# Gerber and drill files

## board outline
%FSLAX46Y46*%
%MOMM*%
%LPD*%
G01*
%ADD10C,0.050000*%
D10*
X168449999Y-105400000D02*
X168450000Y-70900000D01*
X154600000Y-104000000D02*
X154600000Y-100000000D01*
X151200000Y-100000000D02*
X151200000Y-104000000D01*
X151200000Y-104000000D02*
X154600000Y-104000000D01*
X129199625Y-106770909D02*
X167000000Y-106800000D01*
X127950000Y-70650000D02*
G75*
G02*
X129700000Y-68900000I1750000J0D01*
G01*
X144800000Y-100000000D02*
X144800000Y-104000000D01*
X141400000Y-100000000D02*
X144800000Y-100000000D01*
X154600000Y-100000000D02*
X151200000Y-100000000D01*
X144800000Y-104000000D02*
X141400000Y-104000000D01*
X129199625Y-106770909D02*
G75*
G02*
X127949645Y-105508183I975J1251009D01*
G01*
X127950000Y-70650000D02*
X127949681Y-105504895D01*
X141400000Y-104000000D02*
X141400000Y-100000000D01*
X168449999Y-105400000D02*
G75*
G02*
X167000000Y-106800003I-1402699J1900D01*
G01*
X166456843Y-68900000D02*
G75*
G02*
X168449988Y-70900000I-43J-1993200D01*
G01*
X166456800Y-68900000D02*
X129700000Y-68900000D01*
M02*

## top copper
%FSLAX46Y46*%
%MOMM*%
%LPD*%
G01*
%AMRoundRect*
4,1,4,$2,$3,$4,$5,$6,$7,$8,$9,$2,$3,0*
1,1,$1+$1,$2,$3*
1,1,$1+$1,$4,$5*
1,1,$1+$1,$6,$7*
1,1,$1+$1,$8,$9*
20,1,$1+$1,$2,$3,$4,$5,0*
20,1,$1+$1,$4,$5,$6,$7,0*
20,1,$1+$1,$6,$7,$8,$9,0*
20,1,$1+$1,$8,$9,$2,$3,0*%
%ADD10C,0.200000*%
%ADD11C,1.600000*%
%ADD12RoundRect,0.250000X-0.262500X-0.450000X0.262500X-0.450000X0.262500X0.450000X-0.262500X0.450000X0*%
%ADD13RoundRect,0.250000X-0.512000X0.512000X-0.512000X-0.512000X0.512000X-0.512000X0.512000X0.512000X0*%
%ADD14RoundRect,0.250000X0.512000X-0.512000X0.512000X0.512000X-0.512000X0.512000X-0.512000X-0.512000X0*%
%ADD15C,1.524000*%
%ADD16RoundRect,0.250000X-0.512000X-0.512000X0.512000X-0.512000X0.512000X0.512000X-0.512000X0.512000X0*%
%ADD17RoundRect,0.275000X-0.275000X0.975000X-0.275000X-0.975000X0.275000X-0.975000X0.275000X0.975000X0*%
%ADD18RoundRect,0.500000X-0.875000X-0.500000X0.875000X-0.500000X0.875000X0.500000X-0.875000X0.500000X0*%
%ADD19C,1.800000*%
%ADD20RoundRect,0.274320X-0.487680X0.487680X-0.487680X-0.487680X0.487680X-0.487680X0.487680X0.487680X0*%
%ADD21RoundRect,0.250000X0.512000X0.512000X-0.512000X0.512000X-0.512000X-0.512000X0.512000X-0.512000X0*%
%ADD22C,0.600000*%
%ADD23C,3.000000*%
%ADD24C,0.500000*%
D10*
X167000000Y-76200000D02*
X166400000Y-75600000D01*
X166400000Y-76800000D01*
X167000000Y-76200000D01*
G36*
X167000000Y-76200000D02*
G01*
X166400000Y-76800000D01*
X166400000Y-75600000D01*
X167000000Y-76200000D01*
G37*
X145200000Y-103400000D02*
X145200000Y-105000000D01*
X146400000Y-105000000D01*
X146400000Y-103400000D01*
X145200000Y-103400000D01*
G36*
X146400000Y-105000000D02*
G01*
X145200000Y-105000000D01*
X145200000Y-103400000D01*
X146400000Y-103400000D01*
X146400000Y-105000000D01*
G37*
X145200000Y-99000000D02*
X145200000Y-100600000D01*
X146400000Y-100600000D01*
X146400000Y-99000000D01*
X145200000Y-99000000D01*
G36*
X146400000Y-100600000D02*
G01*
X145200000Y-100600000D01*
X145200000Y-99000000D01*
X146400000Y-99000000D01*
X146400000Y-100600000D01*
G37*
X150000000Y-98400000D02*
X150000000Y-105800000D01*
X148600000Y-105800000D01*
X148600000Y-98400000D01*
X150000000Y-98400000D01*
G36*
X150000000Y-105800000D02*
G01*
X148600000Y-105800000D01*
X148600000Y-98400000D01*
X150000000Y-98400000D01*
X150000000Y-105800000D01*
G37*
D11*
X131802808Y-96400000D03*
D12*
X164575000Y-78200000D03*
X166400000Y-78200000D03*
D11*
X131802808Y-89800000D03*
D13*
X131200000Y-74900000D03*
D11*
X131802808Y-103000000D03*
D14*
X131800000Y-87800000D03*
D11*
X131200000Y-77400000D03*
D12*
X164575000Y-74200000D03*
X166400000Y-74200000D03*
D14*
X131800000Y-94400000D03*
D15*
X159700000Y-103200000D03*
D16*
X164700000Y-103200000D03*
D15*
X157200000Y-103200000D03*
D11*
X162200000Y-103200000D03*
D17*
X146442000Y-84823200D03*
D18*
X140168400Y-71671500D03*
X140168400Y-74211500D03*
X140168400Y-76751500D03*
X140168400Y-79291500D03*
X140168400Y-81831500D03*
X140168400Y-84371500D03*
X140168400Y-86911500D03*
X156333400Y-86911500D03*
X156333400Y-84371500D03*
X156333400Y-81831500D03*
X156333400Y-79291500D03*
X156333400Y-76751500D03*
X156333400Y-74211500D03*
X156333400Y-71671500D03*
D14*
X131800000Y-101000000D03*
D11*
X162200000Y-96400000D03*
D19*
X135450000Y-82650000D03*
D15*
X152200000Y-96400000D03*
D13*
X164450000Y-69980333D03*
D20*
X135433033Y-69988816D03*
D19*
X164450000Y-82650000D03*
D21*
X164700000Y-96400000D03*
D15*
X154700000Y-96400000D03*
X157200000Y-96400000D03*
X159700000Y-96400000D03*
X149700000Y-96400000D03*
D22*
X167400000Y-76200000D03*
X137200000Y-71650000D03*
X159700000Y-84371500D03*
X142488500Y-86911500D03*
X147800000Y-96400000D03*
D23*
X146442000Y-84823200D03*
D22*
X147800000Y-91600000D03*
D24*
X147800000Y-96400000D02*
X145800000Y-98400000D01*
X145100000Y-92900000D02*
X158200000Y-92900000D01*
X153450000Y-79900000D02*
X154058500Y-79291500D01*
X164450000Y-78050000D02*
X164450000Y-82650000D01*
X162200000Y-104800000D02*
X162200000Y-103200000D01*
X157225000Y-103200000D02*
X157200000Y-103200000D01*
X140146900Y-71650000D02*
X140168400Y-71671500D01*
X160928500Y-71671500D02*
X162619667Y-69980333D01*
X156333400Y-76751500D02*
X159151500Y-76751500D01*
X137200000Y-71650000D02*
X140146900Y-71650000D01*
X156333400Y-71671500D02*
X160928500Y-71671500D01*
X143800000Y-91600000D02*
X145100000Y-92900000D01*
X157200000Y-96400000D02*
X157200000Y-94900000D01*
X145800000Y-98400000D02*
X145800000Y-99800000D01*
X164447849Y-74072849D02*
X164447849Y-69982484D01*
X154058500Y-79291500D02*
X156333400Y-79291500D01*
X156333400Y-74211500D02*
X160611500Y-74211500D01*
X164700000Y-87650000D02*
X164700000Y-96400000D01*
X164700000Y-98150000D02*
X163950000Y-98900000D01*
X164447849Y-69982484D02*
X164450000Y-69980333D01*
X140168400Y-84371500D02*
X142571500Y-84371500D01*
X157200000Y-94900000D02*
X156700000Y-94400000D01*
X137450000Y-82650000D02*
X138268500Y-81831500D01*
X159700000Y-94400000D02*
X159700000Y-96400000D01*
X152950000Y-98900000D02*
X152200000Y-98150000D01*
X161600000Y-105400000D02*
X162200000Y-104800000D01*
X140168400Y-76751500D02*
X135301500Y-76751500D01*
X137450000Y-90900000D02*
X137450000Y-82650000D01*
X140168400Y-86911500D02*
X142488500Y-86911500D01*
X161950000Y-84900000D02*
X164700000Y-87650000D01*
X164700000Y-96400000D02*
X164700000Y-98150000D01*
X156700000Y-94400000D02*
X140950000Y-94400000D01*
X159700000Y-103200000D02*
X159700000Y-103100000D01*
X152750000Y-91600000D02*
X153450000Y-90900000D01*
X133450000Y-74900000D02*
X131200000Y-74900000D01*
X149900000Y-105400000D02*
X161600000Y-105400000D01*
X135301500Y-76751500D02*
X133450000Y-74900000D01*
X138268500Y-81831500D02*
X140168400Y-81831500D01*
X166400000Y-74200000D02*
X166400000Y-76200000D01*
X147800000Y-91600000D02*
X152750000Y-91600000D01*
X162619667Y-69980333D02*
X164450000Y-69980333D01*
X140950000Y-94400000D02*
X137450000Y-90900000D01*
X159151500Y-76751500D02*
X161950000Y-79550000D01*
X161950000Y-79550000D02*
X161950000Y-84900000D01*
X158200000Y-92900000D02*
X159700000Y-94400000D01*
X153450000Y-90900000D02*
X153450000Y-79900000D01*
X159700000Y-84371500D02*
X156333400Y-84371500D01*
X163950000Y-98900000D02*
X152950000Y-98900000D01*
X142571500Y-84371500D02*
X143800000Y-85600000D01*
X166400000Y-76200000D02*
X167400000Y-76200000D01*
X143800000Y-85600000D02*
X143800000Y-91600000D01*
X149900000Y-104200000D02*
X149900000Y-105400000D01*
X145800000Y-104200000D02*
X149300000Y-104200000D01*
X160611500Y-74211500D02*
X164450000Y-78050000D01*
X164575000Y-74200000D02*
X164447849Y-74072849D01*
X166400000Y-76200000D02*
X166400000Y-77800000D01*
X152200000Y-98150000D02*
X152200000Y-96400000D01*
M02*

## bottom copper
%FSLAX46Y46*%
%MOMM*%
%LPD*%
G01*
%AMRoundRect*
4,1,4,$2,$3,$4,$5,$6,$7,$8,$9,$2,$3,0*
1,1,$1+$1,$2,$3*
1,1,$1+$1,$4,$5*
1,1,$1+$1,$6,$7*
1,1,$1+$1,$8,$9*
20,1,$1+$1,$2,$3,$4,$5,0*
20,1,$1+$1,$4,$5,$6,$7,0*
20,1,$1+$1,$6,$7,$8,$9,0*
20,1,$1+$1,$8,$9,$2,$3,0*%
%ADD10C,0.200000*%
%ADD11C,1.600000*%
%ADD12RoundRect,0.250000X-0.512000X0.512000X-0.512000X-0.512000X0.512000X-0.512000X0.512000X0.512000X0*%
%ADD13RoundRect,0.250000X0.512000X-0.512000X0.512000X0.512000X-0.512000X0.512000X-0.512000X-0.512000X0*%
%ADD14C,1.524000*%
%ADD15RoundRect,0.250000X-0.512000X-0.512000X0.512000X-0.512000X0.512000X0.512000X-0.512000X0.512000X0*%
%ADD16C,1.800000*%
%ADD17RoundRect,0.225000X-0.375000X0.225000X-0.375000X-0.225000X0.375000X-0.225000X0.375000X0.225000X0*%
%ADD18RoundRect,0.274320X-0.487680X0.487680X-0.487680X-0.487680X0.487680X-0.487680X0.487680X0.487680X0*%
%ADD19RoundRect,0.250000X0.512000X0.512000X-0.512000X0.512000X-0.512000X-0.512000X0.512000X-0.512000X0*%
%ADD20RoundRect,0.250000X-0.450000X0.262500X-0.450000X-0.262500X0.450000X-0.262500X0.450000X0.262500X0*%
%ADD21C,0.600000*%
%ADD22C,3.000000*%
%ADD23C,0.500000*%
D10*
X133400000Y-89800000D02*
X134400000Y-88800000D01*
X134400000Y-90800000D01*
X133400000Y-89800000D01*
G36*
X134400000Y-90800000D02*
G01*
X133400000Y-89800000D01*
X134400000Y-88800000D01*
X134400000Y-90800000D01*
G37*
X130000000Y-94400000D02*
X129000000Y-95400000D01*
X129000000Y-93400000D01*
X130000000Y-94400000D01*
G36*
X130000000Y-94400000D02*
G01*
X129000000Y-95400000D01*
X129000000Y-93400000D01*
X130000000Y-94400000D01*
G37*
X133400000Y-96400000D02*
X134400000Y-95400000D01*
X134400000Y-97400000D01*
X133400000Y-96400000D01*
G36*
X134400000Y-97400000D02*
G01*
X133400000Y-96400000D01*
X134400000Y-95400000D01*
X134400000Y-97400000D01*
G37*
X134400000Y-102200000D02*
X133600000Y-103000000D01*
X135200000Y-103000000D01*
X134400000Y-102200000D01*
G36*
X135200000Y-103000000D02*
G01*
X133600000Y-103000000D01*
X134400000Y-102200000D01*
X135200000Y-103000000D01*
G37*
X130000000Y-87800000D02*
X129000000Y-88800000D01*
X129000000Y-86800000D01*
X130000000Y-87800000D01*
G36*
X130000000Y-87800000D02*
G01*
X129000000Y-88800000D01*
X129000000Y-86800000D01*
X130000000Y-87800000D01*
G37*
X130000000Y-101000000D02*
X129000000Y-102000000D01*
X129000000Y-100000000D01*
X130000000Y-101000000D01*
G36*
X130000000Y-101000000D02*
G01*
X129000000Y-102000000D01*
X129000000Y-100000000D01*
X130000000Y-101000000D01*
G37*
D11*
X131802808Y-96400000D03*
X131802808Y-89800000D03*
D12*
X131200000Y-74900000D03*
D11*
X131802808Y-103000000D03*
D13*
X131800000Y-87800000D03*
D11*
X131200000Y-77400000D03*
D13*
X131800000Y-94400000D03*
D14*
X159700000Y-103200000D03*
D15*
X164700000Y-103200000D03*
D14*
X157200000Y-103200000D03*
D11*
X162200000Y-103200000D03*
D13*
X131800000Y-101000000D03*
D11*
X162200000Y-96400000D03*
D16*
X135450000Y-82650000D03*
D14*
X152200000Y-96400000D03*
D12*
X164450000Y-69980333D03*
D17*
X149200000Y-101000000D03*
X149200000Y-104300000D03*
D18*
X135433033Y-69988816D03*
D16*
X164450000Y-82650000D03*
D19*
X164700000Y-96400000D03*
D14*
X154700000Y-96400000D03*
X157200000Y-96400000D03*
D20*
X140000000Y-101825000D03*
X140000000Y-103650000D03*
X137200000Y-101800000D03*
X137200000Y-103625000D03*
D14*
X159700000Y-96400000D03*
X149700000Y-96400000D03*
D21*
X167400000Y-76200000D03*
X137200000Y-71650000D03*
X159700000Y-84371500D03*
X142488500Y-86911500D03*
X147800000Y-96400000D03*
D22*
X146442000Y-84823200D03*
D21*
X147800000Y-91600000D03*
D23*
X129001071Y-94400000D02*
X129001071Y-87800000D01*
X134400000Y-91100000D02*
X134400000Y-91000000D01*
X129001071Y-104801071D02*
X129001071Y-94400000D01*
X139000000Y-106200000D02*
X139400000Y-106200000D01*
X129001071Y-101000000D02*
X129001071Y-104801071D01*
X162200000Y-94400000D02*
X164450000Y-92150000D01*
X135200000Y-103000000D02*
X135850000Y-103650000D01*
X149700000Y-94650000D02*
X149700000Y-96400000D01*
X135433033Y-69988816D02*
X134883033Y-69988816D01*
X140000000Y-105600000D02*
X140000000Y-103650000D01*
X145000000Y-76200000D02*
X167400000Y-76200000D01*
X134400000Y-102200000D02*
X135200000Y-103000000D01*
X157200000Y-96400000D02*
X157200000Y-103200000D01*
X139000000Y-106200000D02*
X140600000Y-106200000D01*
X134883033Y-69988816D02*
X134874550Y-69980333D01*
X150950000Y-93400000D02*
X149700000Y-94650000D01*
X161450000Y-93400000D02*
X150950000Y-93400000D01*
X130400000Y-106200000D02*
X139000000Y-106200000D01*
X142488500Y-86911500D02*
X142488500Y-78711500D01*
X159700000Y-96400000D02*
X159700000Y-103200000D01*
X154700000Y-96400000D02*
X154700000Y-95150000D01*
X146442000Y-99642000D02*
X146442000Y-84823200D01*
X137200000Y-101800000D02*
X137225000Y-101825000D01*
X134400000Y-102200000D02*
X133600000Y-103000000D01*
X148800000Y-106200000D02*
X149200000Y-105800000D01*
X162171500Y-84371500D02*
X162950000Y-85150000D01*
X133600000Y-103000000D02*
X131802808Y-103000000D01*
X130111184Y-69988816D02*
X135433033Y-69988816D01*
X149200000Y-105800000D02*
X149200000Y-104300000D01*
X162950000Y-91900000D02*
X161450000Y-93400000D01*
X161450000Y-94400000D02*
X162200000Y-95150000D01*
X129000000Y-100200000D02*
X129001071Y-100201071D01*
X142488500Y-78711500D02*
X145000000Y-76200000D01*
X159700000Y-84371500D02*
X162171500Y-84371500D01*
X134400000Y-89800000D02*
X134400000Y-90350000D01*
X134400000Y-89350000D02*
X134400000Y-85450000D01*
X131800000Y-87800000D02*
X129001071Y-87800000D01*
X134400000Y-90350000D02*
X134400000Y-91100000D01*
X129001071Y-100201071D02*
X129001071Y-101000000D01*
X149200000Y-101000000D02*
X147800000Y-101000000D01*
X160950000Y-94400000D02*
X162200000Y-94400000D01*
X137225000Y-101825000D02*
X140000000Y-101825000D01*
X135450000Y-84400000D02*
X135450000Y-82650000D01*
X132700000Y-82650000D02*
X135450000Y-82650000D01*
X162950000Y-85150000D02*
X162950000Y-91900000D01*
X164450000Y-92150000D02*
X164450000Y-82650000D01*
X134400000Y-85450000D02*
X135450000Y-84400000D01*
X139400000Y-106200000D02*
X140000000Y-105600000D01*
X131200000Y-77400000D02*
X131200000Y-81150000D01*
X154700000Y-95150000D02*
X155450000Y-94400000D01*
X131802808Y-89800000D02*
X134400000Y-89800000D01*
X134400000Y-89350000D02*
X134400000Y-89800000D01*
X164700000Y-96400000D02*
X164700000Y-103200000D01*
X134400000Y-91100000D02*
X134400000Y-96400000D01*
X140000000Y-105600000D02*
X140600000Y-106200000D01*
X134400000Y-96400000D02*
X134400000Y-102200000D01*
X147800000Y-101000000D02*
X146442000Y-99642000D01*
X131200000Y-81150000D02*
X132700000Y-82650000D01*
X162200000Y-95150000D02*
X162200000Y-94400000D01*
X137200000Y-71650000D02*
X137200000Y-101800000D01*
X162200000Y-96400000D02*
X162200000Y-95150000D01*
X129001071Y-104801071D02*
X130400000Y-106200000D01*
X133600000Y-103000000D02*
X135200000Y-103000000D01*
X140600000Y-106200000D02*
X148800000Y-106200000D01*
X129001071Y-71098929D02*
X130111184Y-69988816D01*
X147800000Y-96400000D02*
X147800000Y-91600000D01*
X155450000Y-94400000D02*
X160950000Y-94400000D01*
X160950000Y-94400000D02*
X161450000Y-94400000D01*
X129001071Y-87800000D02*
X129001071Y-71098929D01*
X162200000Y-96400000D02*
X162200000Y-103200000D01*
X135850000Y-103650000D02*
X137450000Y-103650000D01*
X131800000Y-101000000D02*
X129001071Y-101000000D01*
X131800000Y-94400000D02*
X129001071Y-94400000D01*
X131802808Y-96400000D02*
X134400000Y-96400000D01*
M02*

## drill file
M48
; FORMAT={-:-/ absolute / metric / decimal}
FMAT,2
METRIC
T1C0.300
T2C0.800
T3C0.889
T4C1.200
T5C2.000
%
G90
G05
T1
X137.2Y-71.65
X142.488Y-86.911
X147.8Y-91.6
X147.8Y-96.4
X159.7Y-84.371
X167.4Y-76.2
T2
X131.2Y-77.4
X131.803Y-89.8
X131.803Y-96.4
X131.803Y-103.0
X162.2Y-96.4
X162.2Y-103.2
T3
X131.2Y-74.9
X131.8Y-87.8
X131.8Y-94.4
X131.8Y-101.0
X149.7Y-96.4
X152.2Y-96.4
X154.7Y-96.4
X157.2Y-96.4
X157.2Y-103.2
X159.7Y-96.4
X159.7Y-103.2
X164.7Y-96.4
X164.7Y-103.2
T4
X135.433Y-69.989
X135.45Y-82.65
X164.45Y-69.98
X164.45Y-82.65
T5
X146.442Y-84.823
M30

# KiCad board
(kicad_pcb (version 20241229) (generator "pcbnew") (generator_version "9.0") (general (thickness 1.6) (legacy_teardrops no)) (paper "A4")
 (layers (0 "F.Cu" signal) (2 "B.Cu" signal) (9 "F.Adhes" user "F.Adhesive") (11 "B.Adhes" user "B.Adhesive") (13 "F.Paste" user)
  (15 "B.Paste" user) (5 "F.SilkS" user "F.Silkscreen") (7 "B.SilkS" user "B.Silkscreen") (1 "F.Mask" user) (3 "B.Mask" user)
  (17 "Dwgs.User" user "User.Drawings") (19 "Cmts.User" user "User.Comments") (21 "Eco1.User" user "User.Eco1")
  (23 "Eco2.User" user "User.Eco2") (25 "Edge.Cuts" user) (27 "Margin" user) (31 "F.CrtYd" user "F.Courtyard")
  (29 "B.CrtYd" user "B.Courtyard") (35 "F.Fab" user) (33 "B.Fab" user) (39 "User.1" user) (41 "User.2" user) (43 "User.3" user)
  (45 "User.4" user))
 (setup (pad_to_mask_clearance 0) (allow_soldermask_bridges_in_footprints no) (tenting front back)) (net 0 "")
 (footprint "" (layer "F.Cu") (at 131.802808 96.4 180)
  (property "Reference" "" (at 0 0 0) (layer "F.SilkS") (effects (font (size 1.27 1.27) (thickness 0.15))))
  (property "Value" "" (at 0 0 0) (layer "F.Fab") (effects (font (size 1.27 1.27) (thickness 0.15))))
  (pad "GND" thru_hole circle (at 0 0 90) (size 1.6 1.6) (drill 0.8) (layers "*.Cu" "*.Mask") (remove_unused_layers no)))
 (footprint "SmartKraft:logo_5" (layer "F.Cu") (at 163.6 87)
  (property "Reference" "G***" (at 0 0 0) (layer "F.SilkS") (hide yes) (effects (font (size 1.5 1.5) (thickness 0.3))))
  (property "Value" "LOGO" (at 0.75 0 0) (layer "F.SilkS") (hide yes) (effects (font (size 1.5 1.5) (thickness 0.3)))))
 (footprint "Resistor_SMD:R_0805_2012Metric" (layer "F.Cu") (at 165.4875 78.2)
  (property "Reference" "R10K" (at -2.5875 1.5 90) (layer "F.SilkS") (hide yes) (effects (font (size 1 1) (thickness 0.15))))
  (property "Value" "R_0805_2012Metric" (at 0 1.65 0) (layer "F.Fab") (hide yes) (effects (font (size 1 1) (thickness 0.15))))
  (pad "1" smd roundrect (at -0.9125 0) (size 1.025 1.4) (layers "F.Cu" "F.Mask" "F.Paste") (roundrect_rratio 0.243902))
  (pad "2" smd roundrect (at 0.9125 0) (size 1.025 1.4) (layers "F.Cu" "F.Mask" "F.Paste") (roundrect_rratio 0.243902)))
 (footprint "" (layer "F.Cu") (at 131.802808 89.8 180)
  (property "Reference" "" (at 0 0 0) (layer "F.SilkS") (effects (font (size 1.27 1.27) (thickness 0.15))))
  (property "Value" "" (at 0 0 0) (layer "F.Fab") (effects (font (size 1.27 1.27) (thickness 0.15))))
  (pad "GND" thru_hole circle (at 0 0 90) (size 1.6 1.6) (drill 0.8) (layers "*.Cu" "*.Mask") (remove_unused_layers no)))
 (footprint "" (layer "F.Cu") (at 131.2 74.9 -90)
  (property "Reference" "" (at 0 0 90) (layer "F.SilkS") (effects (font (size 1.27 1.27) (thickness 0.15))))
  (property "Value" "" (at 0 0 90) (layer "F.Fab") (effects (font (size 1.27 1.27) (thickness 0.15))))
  (pad "+" thru_hole roundrect (at 0 0 270) (size 1.524 1.524) (drill 0.889) (layers "*.Cu" "*.Mask") (remove_unused_layers no)
   (roundrect_rratio 0.1640419948)))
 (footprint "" (layer "F.Cu") (at 131.802808 103 180)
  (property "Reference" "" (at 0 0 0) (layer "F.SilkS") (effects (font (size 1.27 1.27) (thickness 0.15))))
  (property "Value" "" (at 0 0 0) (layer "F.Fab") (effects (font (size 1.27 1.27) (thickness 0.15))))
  (pad "GND" thru_hole circle (at 0 0 90) (size 1.6 1.6) (drill 0.8) (layers "*.Cu" "*.Mask") (remove_unused_layers no)))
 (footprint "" (layer "F.Cu") (at 131.8 87.8 180)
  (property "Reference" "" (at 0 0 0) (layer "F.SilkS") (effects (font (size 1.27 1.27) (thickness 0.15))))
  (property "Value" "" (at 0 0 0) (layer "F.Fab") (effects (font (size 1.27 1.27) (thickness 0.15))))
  (pad "+" thru_hole roundrect (at 0 0 90) (size 1.524 1.524) (drill 0.889) (layers "*.Cu" "*.Mask") (remove_unused_layers no)
   (roundrect_rratio 0.1640419948)))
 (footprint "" (layer "F.Cu") (at 131.2 77.4 -90)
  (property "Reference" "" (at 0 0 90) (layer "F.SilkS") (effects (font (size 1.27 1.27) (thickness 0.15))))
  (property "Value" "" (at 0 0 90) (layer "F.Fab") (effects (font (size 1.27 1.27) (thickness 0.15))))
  (pad "GND" thru_hole circle (at 0 0 270) (size 1.6 1.6) (drill 0.8) (layers "*.Cu" "*.Mask") (remove_unused_layers no)))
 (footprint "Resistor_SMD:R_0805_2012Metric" (layer "F.Cu") (at 165.4875 74.2)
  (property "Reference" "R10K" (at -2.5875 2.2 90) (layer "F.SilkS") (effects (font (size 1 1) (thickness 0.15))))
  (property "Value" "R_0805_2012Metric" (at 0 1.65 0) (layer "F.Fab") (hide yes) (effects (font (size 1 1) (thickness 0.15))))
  (pad "1" smd roundrect (at -0.9125 0) (size 1.025 1.4) (layers "F.Cu" "F.Mask" "F.Paste") (roundrect_rratio 0.243902))
  (pad "2" smd roundrect (at 0.9125 0) (size 1.025 1.4) (layers "F.Cu" "F.Mask" "F.Paste") (roundrect_rratio 0.243902)))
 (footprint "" (layer "F.Cu") (at 131.8 94.4 180)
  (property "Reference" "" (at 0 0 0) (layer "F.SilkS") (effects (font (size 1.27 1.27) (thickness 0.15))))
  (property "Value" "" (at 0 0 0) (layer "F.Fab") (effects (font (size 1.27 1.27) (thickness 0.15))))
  (pad "+" thru_hole roundrect (at 0 0 90) (size 1.524 1.524) (drill 0.889) (layers "*.Cu" "*.Mask") (remove_unused_layers no)
   (roundrect_rratio 0.1640419948)))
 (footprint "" (layer "F.Cu") (at 159.7 103.2)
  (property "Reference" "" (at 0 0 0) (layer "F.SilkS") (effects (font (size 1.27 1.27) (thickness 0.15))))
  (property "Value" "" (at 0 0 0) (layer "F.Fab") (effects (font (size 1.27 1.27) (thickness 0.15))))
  (pad "SCL" thru_hole circle (at 0 0) (size 1.524 1.524) (drill 0.889) (layers "*.Cu" "*.Mask") (remove_unused_layers no)))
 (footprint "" (layer "F.Cu") (at 164.7 103.2)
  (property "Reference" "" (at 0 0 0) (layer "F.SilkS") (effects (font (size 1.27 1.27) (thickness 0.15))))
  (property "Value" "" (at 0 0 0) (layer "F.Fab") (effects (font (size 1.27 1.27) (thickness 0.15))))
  (pad "3.3V" thru_hole roundrect (at 0 0) (size 1.524 1.524) (drill 0.889) (layers "*.Cu" "*.Mask") (remove_unused_layers no)
   (roundrect_rratio 0.1640419948)))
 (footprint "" (layer "F.Cu") (at 157.2 103.2)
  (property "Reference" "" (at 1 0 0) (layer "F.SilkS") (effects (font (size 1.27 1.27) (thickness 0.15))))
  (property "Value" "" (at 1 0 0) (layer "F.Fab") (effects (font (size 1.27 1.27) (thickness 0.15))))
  (pad "SDA" thru_hole circle (at 0 0) (size 1.524 1.524) (drill 0.889) (layers "*.Cu" "*.Mask") (remove_unused_layers no)))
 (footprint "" (layer "F.Cu") (at 162.2 103.2)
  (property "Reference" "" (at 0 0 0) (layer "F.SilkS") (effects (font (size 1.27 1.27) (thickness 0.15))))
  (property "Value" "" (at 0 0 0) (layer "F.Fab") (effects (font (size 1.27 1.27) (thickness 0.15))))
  (pad "GND" thru_hole circle (at 0 0) (size 1.6 1.6) (drill 0.8) (layers "*.Cu" "*.Mask") (remove_unused_layers no)))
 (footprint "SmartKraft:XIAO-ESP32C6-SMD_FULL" (layer "F.Cu") (at 148.45 79.27)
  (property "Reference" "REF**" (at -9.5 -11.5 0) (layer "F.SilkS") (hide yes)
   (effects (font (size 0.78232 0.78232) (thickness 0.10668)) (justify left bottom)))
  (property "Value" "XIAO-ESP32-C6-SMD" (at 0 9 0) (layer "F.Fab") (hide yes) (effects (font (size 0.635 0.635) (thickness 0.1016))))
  (pad "" smd circle (at -1.5 -8.62) (size 1.7 1.7) (layers)) (pad "" smd circle (at -1.5 -6.08) (size 1.7 1.7) (layers))
  (pad "" smd circle (at -1.5 -3.54) (size 1.7 1.7) (layers)) (pad "" smd circle (at -1.5 -1) (size 1.7 1.7) (layers))
  (pad "" smd roundrect (at 0.532 5.5532 270) (size 2.5 1.1) (layers) (roundrect_rratio 0.25) (solder_mask_margin 0.0508)
   (thermal_bridge_angle 45))
  (pad "" smd circle (at 0.9474 -1.0568) (size 1.7 1.7) (layers)) (pad "" smd circle (at 1.04 -8.62) (size 1.7 1.7) (layers))
  (pad "" smd circle (at 1.04 -6.08) (size 1.7 1.7) (layers)) (pad "" smd circle (at 1.04 -3.54) (size 1.7 1.7) (layers))
  (pad "+" smd roundrect (at -2.008 5.5532 270) (size 2.5 1.1) (layers "F.Cu" "F.Mask") (roundrect_rratio 0.25) (solder_mask_margin 0.0508)
   (thermal_bridge_angle 45))
  (pad "1" smd roundrect (at -8.2816 -7.5985) (size 2.75 2) (layers "F.Cu" "F.Mask") (roundrect_rratio 0.25) (solder_mask_margin 0.0508)
   (thermal_bridge_angle 45))
  (pad "2" smd roundrect (at -8.2816 -5.0585) (size 2.75 2) (layers "F.Cu" "F.Mask") (roundrect_rratio 0.25) (solder_mask_margin 0.0508)
   (thermal_bridge_angle 45))
  (pad "3" smd roundrect (at -8.2816 -2.5185) (size 2.75 2) (layers "F.Cu" "F.Mask") (roundrect_rratio 0.25) (solder_mask_margin 0.0508)
   (thermal_bridge_angle 45))
  (pad "4" smd roundrect (at -8.2816 0.0215) (size 2.75 2) (layers "F.Cu" "F.Mask") (roundrect_rratio 0.25) (solder_mask_margin 0.0508)
   (thermal_bridge_angle 45))
  (pad "5" smd roundrect (at -8.2816 2.5615) (size 2.75 2) (layers "F.Cu" "F.Mask") (roundrect_rratio 0.25) (solder_mask_margin 0.0508)
   (thermal_bridge_angle 45))
  (pad "6" smd roundrect (at -8.2816 5.1015) (size 2.75 2) (layers "F.Cu" "F.Mask") (roundrect_rratio 0.25) (solder_mask_margin 0.0508)
   (thermal_bridge_angle 45))
  (pad "7" smd roundrect (at -8.2816 7.6415) (size 2.75 2) (layers "F.Cu" "F.Mask") (roundrect_rratio 0.25) (solder_mask_margin 0.0508)
   (thermal_bridge_angle 45))
  (pad "8" smd roundrect (at 7.8834 7.6415) (size 2.75 2) (layers "F.Cu" "F.Mask") (roundrect_rratio 0.25) (solder_mask_margin 0.0508)
   (thermal_bridge_angle 45))
  (pad "9" smd roundrect (at 7.8834 5.1015) (size 2.75 2) (layers "F.Cu" "F.Mask") (roundrect_rratio 0.25) (solder_mask_margin 0.0508)
   (thermal_bridge_angle 45))
  (pad "10" smd roundrect (at 7.8834 2.5615) (size 2.75 2) (layers "F.Cu" "F.Mask") (roundrect_rratio 0.25) (solder_mask_margin 0.0508)
   (thermal_bridge_angle 45))
  (pad "11" smd roundrect (at 7.8834 0.0215) (size 2.75 2) (layers "F.Cu" "F.Mask") (roundrect_rratio 0.25) (solder_mask_margin 0.0508)
   (thermal_bridge_angle 45))
  (pad "12" smd roundrect (at 7.8834 -2.5185) (size 2.75 2) (layers "F.Cu" "F.Mask") (roundrect_rratio 0.25) (solder_mask_margin 0.0508)
   (thermal_bridge_angle 45))
  (pad "13" smd roundrect (at 7.8834 -5.0585) (size 2.75 2) (layers "F.Cu" "F.Mask") (roundrect_rratio 0.25) (solder_mask_margin 0.0508)
   (thermal_bridge_angle 45))
  (pad "14" smd roundrect (at 7.8834 -7.5985) (size 2.75 2) (layers "F.Cu" "F.Mask") (roundrect_rratio 0.25) (solder_mask_margin 0.0508)
   (thermal_bridge_angle 45)))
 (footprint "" (layer "F.Cu") (at 131.8 101 180)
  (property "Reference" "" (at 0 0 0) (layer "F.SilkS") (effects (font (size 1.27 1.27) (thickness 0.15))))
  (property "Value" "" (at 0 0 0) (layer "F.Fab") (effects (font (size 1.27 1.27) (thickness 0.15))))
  (pad "+" thru_hole roundrect (at 0 0 90) (size 1.524 1.524) (drill 0.889) (layers "*.Cu" "*.Mask") (remove_unused_layers no)
   (roundrect_rratio 0.1640419948)))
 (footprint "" (layer "B.Cu") (at 162.2 96.4)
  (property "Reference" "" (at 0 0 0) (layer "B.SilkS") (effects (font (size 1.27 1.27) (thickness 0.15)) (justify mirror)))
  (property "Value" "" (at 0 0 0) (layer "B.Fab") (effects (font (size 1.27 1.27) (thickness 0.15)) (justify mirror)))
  (pad "GND" thru_hole circle (at 0 0) (size 1.6 1.6) (drill 0.8) (layers "*.Cu" "*.Mask") (remove_unused_layers no)))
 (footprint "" (layer "B.Cu") (at 135.45 82.65 -90)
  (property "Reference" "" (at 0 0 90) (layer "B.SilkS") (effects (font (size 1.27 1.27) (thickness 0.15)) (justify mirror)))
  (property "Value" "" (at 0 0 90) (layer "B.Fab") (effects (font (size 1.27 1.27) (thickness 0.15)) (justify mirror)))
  (pad "GND" thru_hole circle (at 0 0 270) (size 1.8 1.8) (drill 1.2) (layers "*.Cu" "*.Mask") (remove_unused_layers no)))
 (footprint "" (layer "B.Cu") (at 152.2 96.4)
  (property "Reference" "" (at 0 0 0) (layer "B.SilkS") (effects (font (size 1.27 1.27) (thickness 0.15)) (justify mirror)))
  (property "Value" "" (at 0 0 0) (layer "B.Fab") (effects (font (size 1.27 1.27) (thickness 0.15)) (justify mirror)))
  (pad "CS" thru_hole circle (at 0 0) (size 1.524 1.524) (drill 0.889) (layers "*.Cu" "*.Mask") (remove_unused_layers no)))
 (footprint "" (layer "B.Cu") (at 164.45 69.980333 -90)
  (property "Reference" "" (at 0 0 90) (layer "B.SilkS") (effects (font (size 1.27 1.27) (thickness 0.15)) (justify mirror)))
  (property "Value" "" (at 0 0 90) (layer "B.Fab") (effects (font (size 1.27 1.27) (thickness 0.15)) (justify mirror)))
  (pad "+" thru_hole roundrect (at 0 0 270) (size 1.524 1.524) (drill 1.2) (layers "*.Cu" "*.Mask") (remove_unused_layers no)
   (roundrect_rratio 0.1640419948)))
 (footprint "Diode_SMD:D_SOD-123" (layer "B.Cu") (at 149.2 102.65 -90)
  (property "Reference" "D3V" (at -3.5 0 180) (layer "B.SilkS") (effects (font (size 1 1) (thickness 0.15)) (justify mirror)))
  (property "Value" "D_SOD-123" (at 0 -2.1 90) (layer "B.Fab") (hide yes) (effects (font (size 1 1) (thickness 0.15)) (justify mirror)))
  (pad "1" smd roundrect (at -1.65 0 270) (size 0.9 1.2) (layers "B.Cu" "B.Mask" "B.Paste") (roundrect_rratio 0.25))
  (pad "2" smd roundrect (at 1.65 0 270) (size 0.9 1.2) (layers "B.Cu" "B.Mask" "B.Paste") (roundrect_rratio 0.25)))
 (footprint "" (layer "B.Cu") (at 135.433033 69.988816 -90)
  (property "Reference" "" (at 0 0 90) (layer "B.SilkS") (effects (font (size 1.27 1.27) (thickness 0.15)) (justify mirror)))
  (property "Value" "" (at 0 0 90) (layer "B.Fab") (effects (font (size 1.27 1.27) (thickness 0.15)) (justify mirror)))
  (pad "+" thru_hole roundrect (at 0 0 270) (size 1.524 1.524) (drill 1.2) (layers "*.Cu" "*.Mask") (remove_unused_layers no)
   (roundrect_rratio 0.18)))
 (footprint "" (layer "B.Cu") (at 164.45 82.65 -90)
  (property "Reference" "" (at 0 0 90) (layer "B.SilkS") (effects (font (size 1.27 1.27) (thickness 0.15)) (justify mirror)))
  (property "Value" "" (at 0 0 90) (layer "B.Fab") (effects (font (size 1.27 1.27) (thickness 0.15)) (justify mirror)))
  (pad "GND" thru_hole circle (at 0 0 270) (size 1.8 1.8) (drill 1.2) (layers "*.Cu" "*.Mask") (remove_unused_layers no)))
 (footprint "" (layer "B.Cu") (at 164.7 96.4 -90)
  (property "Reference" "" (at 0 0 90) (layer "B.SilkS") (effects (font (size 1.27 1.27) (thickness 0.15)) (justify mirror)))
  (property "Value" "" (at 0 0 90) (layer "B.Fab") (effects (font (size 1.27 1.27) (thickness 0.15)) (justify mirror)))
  (pad "3.3V" thru_hole roundrect (at 0 0 180) (size 1.524 1.524) (drill 0.889) (layers "*.Cu" "*.Mask") (remove_unused_layers no)
   (roundrect_rratio 0.1640419948)))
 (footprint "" (layer "B.Cu") (at 154.7 96.4)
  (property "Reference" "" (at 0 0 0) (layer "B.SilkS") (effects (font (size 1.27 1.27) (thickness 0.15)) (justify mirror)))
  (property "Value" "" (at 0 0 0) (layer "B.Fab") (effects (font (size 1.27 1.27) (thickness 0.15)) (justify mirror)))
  (pad "SDO" thru_hole circle (at 0 0) (size 1.524 1.524) (drill 0.889) (layers "*.Cu" "*.Mask") (remove_unused_layers no)))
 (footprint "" (layer "B.Cu") (at 157.2 96.4)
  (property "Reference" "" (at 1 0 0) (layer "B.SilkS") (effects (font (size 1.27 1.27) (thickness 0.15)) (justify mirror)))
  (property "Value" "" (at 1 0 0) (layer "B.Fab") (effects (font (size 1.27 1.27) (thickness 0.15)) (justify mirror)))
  (pad "SDA" thru_hole circle (at 0 0) (size 1.524 1.524) (drill 0.889) (layers "*.Cu" "*.Mask") (remove_unused_layers no)))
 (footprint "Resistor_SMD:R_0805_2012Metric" (layer "B.Cu") (at 140 102.7375 -90)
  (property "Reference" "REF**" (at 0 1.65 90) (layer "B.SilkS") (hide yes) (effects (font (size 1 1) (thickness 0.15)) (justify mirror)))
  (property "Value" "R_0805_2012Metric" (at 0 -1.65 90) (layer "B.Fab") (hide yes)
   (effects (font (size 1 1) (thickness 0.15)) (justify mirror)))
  (pad "1" smd roundrect (at -0.9125 0 270) (size 1.025 1.4) (layers "B.Cu" "B.Mask" "B.Paste") (roundrect_rratio 0.243902))
  (pad "2" smd roundrect (at 0.9125 0 270) (size 1.025 1.4) (layers "B.Cu" "B.Mask" "B.Paste") (roundrect_rratio 0.243902)))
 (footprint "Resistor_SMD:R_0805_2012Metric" (layer "B.Cu") (at 137.2 102.7125 -90)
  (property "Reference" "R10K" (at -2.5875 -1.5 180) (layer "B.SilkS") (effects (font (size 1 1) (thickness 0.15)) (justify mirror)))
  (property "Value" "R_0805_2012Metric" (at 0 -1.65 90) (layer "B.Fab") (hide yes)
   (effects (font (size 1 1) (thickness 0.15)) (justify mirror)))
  (pad "1" smd roundrect (at -0.9125 0 270) (size 1.025 1.4) (layers "B.Cu" "B.Mask" "B.Paste") (roundrect_rratio 0.243902))
  (pad "2" smd roundrect (at 0.9125 0 270) (size 1.025 1.4) (layers "B.Cu" "B.Mask" "B.Paste") (roundrect_rratio 0.243902)))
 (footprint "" (layer "B.Cu") (at 159.7 96.4)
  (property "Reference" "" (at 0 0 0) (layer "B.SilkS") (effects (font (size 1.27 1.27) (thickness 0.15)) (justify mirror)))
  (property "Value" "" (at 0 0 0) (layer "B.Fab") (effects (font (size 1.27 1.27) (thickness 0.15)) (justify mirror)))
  (pad "SCL" thru_hole circle (at 0 0) (size 1.524 1.524) (drill 0.889) (layers "*.Cu" "*.Mask") (remove_unused_layers no)))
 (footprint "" (layer "B.Cu") (at 149.7 96.4)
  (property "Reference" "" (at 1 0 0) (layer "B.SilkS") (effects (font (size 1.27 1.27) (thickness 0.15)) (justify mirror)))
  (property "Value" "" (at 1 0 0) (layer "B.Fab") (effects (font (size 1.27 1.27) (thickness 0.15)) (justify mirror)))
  (pad "INT" thru_hole circle (at 0 0) (size 1.524 1.524) (drill 0.889) (layers "*.Cu" "*.Mask") (remove_unused_layers no)))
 (gr_poly (pts (xy 167 76.2) (xy 166.4 75.6) (xy 166.4 76.8)) (stroke (width 0.2) (type solid)) (fill yes) (layer "F.Cu"))
 (gr_poly
  (pts (xy 145.2 103.4) (xy 145.2 105) (xy 146.4 105) (xy 146.4 103.4)) (stroke (width 0.2) (type solid)) (fill yes)
  (layers "F.Cu" "F.Mask"))
 (gr_poly
  (pts (xy 145.2 99) (xy 145.2 100.6) (xy 146.4 100.6) (xy 146.4 99)) (stroke (width 0.2) (type solid)) (fill yes) (layers "F.Cu" "F.Mask"))
 (gr_poly
  (pts (xy 150 98.4) (xy 150 105.8) (xy 148.6 105.8) (xy 148.6 98.4)) (stroke (width 0.2) (type solid)) (fill yes) (layers "F.Cu" "F.Mask"))
 (gr_poly (pts (xy 133.4 89.8) (xy 134.4 88.8) (xy 134.4 90.8)) (stroke (width 0.2) (type solid)) (fill yes) (layer "B.Cu"))
 (gr_poly (pts (xy 130 94.4) (xy 129 95.4) (xy 129 93.4)) (stroke (width 0.2) (type solid)) (fill yes) (layer "B.Cu"))
 (gr_poly (pts (xy 133.4 96.4) (xy 134.4 95.4) (xy 134.4 97.4)) (stroke (width 0.2) (type solid)) (fill yes) (layer "B.Cu"))
 (gr_poly (pts (xy 134.4 102.2) (xy 133.6 103) (xy 135.2 103)) (stroke (width 0.2) (type solid)) (fill yes) (layer "B.Cu"))
 (gr_poly (pts (xy 130 87.8) (xy 129 88.8) (xy 129 86.8)) (stroke (width 0.2) (type solid)) (fill yes) (layer "B.Cu"))
 (gr_poly (pts (xy 130 101) (xy 129 102) (xy 129 100)) (stroke (width 0.2) (type solid)) (fill yes) (layer "B.Cu"))
 (gr_line (start 168.449999 105.4) (end 168.45 70.9) (stroke (width 0.05) (type default)) (layer "Edge.Cuts"))
 (gr_line (start 154.6 104) (end 154.6 100) (stroke (width 0.05) (type default)) (layer "Edge.Cuts"))
 (gr_line (start 151.2 100) (end 151.2 104) (stroke (width 0.05) (type default)) (layer "Edge.Cuts"))
 (gr_line (start 151.2 104) (end 154.6 104) (stroke (width 0.05) (type default)) (layer "Edge.Cuts"))
 (gr_line (start 129.199625 106.770909) (end 167 106.8) (stroke (width 0.05) (type default)) (layer "Edge.Cuts"))
 (gr_arc (start 127.95 70.65) (mid 128.462563 69.412563) (end 129.7 68.9) (stroke (width 0.05) (type default)) (layer "Edge.Cuts"))
 (gr_line (start 144.8 100) (end 144.8 104) (stroke (width 0.05) (type default)) (layer "Edge.Cuts"))
 (gr_line (start 141.4 100) (end 144.8 100) (stroke (width 0.05) (type default)) (layer "Edge.Cuts"))
 (gr_line (start 154.6 100) (end 151.2 100) (stroke (width 0.05) (type default)) (layer "Edge.Cuts"))
 (gr_line (start 144.8 104) (end 141.4 104) (stroke (width 0.05) (type default)) (layer "Edge.Cuts"))
 (gr_arc (start 129.199625 106.770909) (mid 128.311535 106.4) (end 127.949681 105.508183) (stroke (width 0.05) (type default))
  (layer "Edge.Cuts"))
 (gr_line (start 127.95 70.65) (end 127.949681 105.504895) (stroke (width 0.05) (type default)) (layer "Edge.Cuts"))
 (gr_line (start 141.4 104) (end 141.4 100) (stroke (width 0.05) (type default)) (layer "Edge.Cuts"))
 (gr_arc (start 168.449999 105.4) (mid 168.021618 106.407212) (end 167 106.8) (stroke (width 0.05) (type default)) (layer "Edge.Cuts"))
 (gr_arc (start 166.456843 68.9) (mid 167.868639 69.486203) (end 168.45 70.9) (stroke (width 0.05) (type default)) (layer "Edge.Cuts"))
 (gr_line (start 166.4568 68.9) (end 129.7 68.9) (stroke (width 0.05) (type default)) (layer "Edge.Cuts"))
 (segment (start 147.8 96.4) (end 145.8 98.4) (width 0.5) (layer "F.Cu") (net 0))
 (segment (start 145.1 92.9) (end 158.2 92.9) (width 0.5) (layer "F.Cu") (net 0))
 (segment (start 153.45 79.9) (end 154.0585 79.2915) (width 0.5) (layer "F.Cu") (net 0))
 (segment (start 164.45 78.05) (end 164.45 82.65) (width 0.5) (layer "F.Cu") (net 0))
 (segment (start 162.2 104.8) (end 162.2 103.2) (width 0.5) (layer "F.Cu") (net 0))
 (segment (start 157.225 103.2) (end 157.2 103.2) (width 0.5) (layer "F.Cu") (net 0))
 (segment (start 140.1469 71.65) (end 140.1684 71.6715) (width 0.5) (layer "F.Cu") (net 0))
 (segment (start 160.9285 71.6715) (end 162.619667 69.980333) (width 0.5) (layer "F.Cu") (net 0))
 (segment (start 156.3334 76.7515) (end 159.1515 76.7515) (width 0.5) (layer "F.Cu") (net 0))
 (segment (start 137.2 71.65) (end 140.1469 71.65) (width 0.5) (layer "F.Cu") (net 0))
 (segment (start 156.3334 71.6715) (end 160.9285 71.6715) (width 0.5) (layer "F.Cu") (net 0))
 (segment (start 143.8 91.6) (end 145.1 92.9) (width 0.5) (layer "F.Cu") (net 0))
 (segment (start 157.2 96.4) (end 157.2 94.9) (width 0.5) (layer "F.Cu") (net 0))
 (segment (start 145.8 98.4) (end 145.8 99.8) (width 0.5) (layer "F.Cu") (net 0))
 (segment (start 164.447849 74.072849) (end 164.447849 69.982484) (width 0.5) (layer "F.Cu") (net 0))
 (segment (start 154.0585 79.2915) (end 156.3334 79.2915) (width 0.5) (layer "F.Cu") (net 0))
 (segment (start 156.3334 74.2115) (end 160.6115 74.2115) (width 0.5) (layer "F.Cu") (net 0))
 (segment (start 164.7 87.65) (end 164.7 96.4) (width 0.5) (layer "F.Cu") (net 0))
 (segment (start 164.7 98.15) (end 163.95 98.9) (width 0.5) (layer "F.Cu") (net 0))
 (segment (start 164.447849 69.982484) (end 164.45 69.980333) (width 0.5) (layer "F.Cu") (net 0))
 (segment (start 140.1684 84.3715) (end 142.5715 84.3715) (width 0.5) (layer "F.Cu") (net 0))
 (segment (start 157.2 94.9) (end 156.7 94.4) (width 0.5) (layer "F.Cu") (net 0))
 (segment (start 137.45 82.65) (end 138.2685 81.8315) (width 0.5) (layer "F.Cu") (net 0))
 (segment (start 159.7 94.4) (end 159.7 96.4) (width 0.5) (layer "F.Cu") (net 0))
 (segment (start 152.95 98.9) (end 152.2 98.15) (width 0.5) (layer "F.Cu") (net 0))
 (segment (start 161.6 105.4) (end 162.2 104.8) (width 0.5) (layer "F.Cu") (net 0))
 (segment (start 140.1684 76.7515) (end 135.3015 76.7515) (width 0.5) (layer "F.Cu") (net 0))
 (segment (start 137.45 90.9) (end 137.45 82.65) (width 0.5) (layer "F.Cu") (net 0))
 (segment (start 140.1684 86.9115) (end 142.4885 86.9115) (width 0.5) (layer "F.Cu") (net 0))
 (segment (start 161.95 84.9) (end 164.7 87.65) (width 0.5) (layer "F.Cu") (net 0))
 (segment (start 164.7 96.4) (end 164.7 98.15) (width 0.5) (layer "F.Cu") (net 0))
 (segment (start 156.7 94.4) (end 140.95 94.4) (width 0.5) (layer "F.Cu") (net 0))
 (segment (start 159.7 103.2) (end 159.7 103.1) (width 0.5) (layer "F.Cu") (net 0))
 (segment (start 152.75 91.6) (end 153.45 90.9) (width 0.5) (layer "F.Cu") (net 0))
 (segment (start 133.45 74.9) (end 131.2 74.9) (width 0.5) (layer "F.Cu") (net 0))
 (segment (start 149.9 105.4) (end 161.6 105.4) (width 0.5) (layer "F.Cu") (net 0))
 (segment (start 135.3015 76.7515) (end 133.45 74.9) (width 0.5) (layer "F.Cu") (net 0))
 (segment (start 138.2685 81.8315) (end 140.1684 81.8315) (width 0.5) (layer "F.Cu") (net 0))
 (segment (start 166.4 74.2) (end 166.4 76.2) (width 0.5) (layer "F.Cu") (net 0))
 (segment (start 147.8 91.6) (end 152.75 91.6) (width 0.5) (layer "F.Cu") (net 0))
 (segment (start 162.619667 69.980333) (end 164.45 69.980333) (width 0.5) (layer "F.Cu") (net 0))
 (segment (start 140.95 94.4) (end 137.45 90.9) (width 0.5) (layer "F.Cu") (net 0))
 (segment (start 159.1515 76.7515) (end 161.95 79.55) (width 0.5) (layer "F.Cu") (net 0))
 (segment (start 161.95 79.55) (end 161.95 84.9) (width 0.5) (layer "F.Cu") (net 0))
 (segment (start 158.2 92.9) (end 159.7 94.4) (width 0.5) (layer "F.Cu") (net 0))
 (segment (start 153.45 90.9) (end 153.45 79.9) (width 0.5) (layer "F.Cu") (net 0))
 (segment (start 159.7 84.3715) (end 156.3334 84.3715) (width 0.5) (layer "F.Cu") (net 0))
 (segment (start 163.95 98.9) (end 152.95 98.9) (width 0.5) (layer "F.Cu") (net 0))
 (segment (start 142.5715 84.3715) (end 143.8 85.6) (width 0.5) (layer "F.Cu") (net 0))
 (segment (start 166.4 76.2) (end 167.4 76.2) (width 0.5) (layer "F.Cu") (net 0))
 (segment (start 143.8 85.6) (end 143.8 91.6) (width 0.5) (layer "F.Cu") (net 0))
 (segment (start 149.9 104.2) (end 149.9 105.4) (width 0.5) (layer "F.Cu") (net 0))
 (segment (start 145.8 104.2) (end 149.3 104.2) (width 0.5) (layer "F.Cu") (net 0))
 (segment (start 160.6115 74.2115) (end 164.45 78.05) (width 0.5) (layer "F.Cu") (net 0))
 (segment (start 164.575 74.2) (end 164.447849 74.072849) (width 0.5) (layer "F.Cu") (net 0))
 (segment (start 166.4 76.2) (end 166.4 77.8) (width 0.5) (layer "F.Cu") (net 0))
 (segment (start 152.2 98.15) (end 152.2 96.4) (width 0.5) (layer "F.Cu") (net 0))
 (via (at 167.4 76.2) (size 0.6) (drill 0.3) (layers "F.Cu" "B.Cu") (tenting none) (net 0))
 (via (at 137.2 71.65) (size 0.6) (drill 0.3) (layers "F.Cu" "B.Cu") (tenting none) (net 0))
 (via (at 159.7 84.3715) (size 0.6) (drill 0.3) (layers "F.Cu" "B.Cu") (tenting none) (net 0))
 (via (at 142.4885 86.9115) (size 0.6) (drill 0.3) (layers "F.Cu" "B.Cu") (tenting none) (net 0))
 (via (at 147.8 96.4) (size 0.6) (drill 0.3) (layers "F.Cu" "B.Cu") (tenting none) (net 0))
 (via (at 146.442 84.8232) (size 3) (drill 2) (layers "F.Cu" "B.Cu") (tenting none) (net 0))
 (via (at 147.8 91.6) (size 0.6) (drill 0.3) (layers "F.Cu" "B.Cu") (tenting none) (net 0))
 (segment (start 129.001071 94.4) (end 129.001071 87.8) (width 0.5) (layer "B.Cu") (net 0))
 (segment (start 134.4 91.1) (end 134.4 91) (width 0.5) (layer "B.Cu") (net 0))
 (segment (start 129.001071 104.801071) (end 129.001071 94.4) (width 0.5) (layer "B.Cu") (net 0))
 (segment (start 139 106.2) (end 139.4 106.2) (width 0.5) (layer "B.Cu") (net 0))
 (segment (start 129.001071 101) (end 129.001071 104.801071) (width 0.5) (layer "B.Cu") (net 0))
 (segment (start 162.2 94.4) (end 164.45 92.15) (width 0.5) (layer "B.Cu") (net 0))
 (segment (start 135.2 103) (end 135.85 103.65) (width 0.5) (layer "B.Cu") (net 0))
 (segment (start 149.7 94.65) (end 149.7 96.4) (width 0.5) (layer "B.Cu") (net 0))
 (segment (start 135.433033 69.988816) (end 134.883033 69.988816) (width 0.5) (layer "B.Cu") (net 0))
 (segment (start 140 105.6) (end 140 103.65) (width 0.5) (layer "B.Cu") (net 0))
 (segment (start 145 76.2) (end 167.4 76.2) (width 0.5) (layer "B.Cu") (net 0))
 (segment (start 134.4 102.2) (end 135.2 103) (width 0.5) (layer "B.Cu") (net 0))
 (segment (start 157.2 96.4) (end 157.2 103.2) (width 0.5) (layer "B.Cu") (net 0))
 (segment (start 139 106.2) (end 140.6 106.2) (width 0.5) (layer "B.Cu") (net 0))
 (segment (start 134.883033 69.988816) (end 134.87455 69.980333) (width 0.5) (layer "B.Cu") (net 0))
 (segment (start 150.95 93.4) (end 149.7 94.65) (width 0.5) (layer "B.Cu") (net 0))
 (segment (start 161.45 93.4) (end 150.95 93.4) (width 0.5) (layer "B.Cu") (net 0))
 (segment (start 130.4 106.2) (end 139 106.2) (width 0.5) (layer "B.Cu") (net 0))
 (segment (start 142.4885 86.9115) (end 142.4885 78.7115) (width 0.5) (layer "B.Cu") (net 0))
 (segment (start 159.7 96.4) (end 159.7 103.2) (width 0.5) (layer "B.Cu") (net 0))
 (segment (start 154.7 96.4) (end 154.7 95.15) (width 0.5) (layer "B.Cu") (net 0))
 (segment (start 146.442 99.642) (end 146.442 84.8232) (width 0.5) (layer "B.Cu") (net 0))
 (segment (start 137.2 101.8) (end 137.225 101.825) (width 0.5) (layer "B.Cu") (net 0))
 (segment (start 134.4 102.2) (end 133.6 103) (width 0.5) (layer "B.Cu") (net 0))
 (segment (start 148.8 106.2) (end 149.2 105.8) (width 0.5) (layer "B.Cu") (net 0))
 (segment (start 162.1715 84.3715) (end 162.95 85.15) (width 0.5) (layer "B.Cu") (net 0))
 (segment (start 133.6 103) (end 131.802808 103) (width 0.5) (layer "B.Cu") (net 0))
 (segment (start 130.111184 69.988816) (end 135.433033 69.988816) (width 0.5) (layer "B.Cu") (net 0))
 (segment (start 149.2 105.8) (end 149.2 104.3) (width 0.5) (layer "B.Cu") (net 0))
 (segment (start 162.95 91.9) (end 161.45 93.4) (width 0.5) (layer "B.Cu") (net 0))
 (segment (start 161.45 94.4) (end 162.2 95.15) (width 0.5) (layer "B.Cu") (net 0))
 (segment (start 129 100.2) (end 129.001071 100.201071) (width 0.5) (layer "B.Cu") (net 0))
 (segment (start 142.4885 78.7115) (end 145 76.2) (width 0.5) (layer "B.Cu") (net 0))
 (segment (start 159.7 84.3715) (end 162.1715 84.3715) (width 0.5) (layer "B.Cu") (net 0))
 (segment (start 134.4 89.8) (end 134.4 90.35) (width 0.5) (layer "B.Cu") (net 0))
 (segment (start 134.4 89.35) (end 134.4 85.45) (width 0.5) (layer "B.Cu") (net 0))
 (segment (start 131.8 87.8) (end 129.001071 87.8) (width 0.5) (layer "B.Cu") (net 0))
 (segment (start 134.4 90.35) (end 134.4 91.1) (width 0.5) (layer "B.Cu") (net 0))
 (segment (start 129.001071 100.201071) (end 129.001071 101) (width 0.5) (layer "B.Cu") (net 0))
 (segment (start 149.2 101) (end 147.8 101) (width 0.5) (layer "B.Cu") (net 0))
 (segment (start 160.95 94.4) (end 162.2 94.4) (width 0.5) (layer "B.Cu") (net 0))
 (segment (start 137.225 101.825) (end 140 101.825) (width 0.5) (layer "B.Cu") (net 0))
 (segment (start 135.45 84.4) (end 135.45 82.65) (width 0.5) (layer "B.Cu") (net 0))
 (segment (start 132.7 82.65) (end 135.45 82.65) (width 0.5) (layer "B.Cu") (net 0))
 (segment (start 162.95 85.15) (end 162.95 91.9) (width 0.5) (layer "B.Cu") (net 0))
 (segment (start 164.45 92.15) (end 164.45 82.65) (width 0.5) (layer "B.Cu") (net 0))
 (segment (start 134.4 85.45) (end 135.45 84.4) (width 0.5) (layer "B.Cu") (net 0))
 (segment (start 139.4 106.2) (end 140 105.6) (width 0.5) (layer "B.Cu") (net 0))
 (segment (start 131.2 77.4) (end 131.2 81.15) (width 0.5) (layer "B.Cu") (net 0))
 (segment (start 154.7 95.15) (end 155.45 94.4) (width 0.5) (layer "B.Cu") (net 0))
 (segment (start 131.802808 89.8) (end 134.4 89.8) (width 0.5) (layer "B.Cu") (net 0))
 (segment (start 134.4 89.35) (end 134.4 89.8) (width 0.5) (layer "B.Cu") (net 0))
 (segment (start 164.7 96.4) (end 164.7 103.2) (width 0.5) (layer "B.Cu") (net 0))
 (segment (start 134.4 91.1) (end 134.4 96.4) (width 0.5) (layer "B.Cu") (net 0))
 (segment (start 140 105.6) (end 140.6 106.2) (width 0.5) (layer "B.Cu") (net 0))
 (segment (start 134.4 96.4) (end 134.4 102.2) (width 0.5) (layer "B.Cu") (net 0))
 (segment (start 147.8 101) (end 146.442 99.642) (width 0.5) (layer "B.Cu") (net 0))
 (segment (start 131.2 81.15) (end 132.7 82.65) (width 0.5) (layer "B.Cu") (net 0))
 (segment (start 162.2 95.15) (end 162.2 94.4) (width 0.5) (layer "B.Cu") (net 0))
 (segment (start 137.2 71.65) (end 137.2 101.8) (width 0.5) (layer "B.Cu") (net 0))
 (segment (start 162.2 96.4) (end 162.2 95.15) (width 0.5) (layer "B.Cu") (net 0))
 (segment (start 129.001071 104.801071) (end 130.4 106.2) (width 0.5) (layer "B.Cu") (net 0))
 (segment (start 133.6 103) (end 135.2 103) (width 0.5) (layer "B.Cu") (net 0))
 (segment (start 140.6 106.2) (end 148.8 106.2) (width 0.5) (layer "B.Cu") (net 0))
 (segment (start 129.001071 71.098929) (end 130.111184 69.988816) (width 0.5) (layer "B.Cu") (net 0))
 (segment (start 147.8 96.4) (end 147.8 91.6) (width 0.5) (layer "B.Cu") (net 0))
 (segment (start 155.45 94.4) (end 160.95 94.4) (width 0.5) (layer "B.Cu") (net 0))
 (segment (start 160.95 94.4) (end 161.45 94.4) (width 0.5) (layer "B.Cu") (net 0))
 (segment (start 129.001071 87.8) (end 129.001071 71.098929) (width 0.5) (layer "B.Cu") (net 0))
 (segment (start 162.2 96.4) (end 162.2 103.2) (width 0.5) (layer "B.Cu") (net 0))
 (segment (start 135.85 103.65) (end 137.45 103.65) (width 0.5) (layer "B.Cu") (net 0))
 (segment (start 131.8 101) (end 129.001071 101) (width 0.5) (layer "B.Cu") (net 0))
 (segment (start 131.8 94.4) (end 129.001071 94.4) (width 0.5) (layer "B.Cu") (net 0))
 (segment (start 131.802808 96.4) (end 134.4 96.4) (width 0.5) (layer "B.Cu") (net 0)))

